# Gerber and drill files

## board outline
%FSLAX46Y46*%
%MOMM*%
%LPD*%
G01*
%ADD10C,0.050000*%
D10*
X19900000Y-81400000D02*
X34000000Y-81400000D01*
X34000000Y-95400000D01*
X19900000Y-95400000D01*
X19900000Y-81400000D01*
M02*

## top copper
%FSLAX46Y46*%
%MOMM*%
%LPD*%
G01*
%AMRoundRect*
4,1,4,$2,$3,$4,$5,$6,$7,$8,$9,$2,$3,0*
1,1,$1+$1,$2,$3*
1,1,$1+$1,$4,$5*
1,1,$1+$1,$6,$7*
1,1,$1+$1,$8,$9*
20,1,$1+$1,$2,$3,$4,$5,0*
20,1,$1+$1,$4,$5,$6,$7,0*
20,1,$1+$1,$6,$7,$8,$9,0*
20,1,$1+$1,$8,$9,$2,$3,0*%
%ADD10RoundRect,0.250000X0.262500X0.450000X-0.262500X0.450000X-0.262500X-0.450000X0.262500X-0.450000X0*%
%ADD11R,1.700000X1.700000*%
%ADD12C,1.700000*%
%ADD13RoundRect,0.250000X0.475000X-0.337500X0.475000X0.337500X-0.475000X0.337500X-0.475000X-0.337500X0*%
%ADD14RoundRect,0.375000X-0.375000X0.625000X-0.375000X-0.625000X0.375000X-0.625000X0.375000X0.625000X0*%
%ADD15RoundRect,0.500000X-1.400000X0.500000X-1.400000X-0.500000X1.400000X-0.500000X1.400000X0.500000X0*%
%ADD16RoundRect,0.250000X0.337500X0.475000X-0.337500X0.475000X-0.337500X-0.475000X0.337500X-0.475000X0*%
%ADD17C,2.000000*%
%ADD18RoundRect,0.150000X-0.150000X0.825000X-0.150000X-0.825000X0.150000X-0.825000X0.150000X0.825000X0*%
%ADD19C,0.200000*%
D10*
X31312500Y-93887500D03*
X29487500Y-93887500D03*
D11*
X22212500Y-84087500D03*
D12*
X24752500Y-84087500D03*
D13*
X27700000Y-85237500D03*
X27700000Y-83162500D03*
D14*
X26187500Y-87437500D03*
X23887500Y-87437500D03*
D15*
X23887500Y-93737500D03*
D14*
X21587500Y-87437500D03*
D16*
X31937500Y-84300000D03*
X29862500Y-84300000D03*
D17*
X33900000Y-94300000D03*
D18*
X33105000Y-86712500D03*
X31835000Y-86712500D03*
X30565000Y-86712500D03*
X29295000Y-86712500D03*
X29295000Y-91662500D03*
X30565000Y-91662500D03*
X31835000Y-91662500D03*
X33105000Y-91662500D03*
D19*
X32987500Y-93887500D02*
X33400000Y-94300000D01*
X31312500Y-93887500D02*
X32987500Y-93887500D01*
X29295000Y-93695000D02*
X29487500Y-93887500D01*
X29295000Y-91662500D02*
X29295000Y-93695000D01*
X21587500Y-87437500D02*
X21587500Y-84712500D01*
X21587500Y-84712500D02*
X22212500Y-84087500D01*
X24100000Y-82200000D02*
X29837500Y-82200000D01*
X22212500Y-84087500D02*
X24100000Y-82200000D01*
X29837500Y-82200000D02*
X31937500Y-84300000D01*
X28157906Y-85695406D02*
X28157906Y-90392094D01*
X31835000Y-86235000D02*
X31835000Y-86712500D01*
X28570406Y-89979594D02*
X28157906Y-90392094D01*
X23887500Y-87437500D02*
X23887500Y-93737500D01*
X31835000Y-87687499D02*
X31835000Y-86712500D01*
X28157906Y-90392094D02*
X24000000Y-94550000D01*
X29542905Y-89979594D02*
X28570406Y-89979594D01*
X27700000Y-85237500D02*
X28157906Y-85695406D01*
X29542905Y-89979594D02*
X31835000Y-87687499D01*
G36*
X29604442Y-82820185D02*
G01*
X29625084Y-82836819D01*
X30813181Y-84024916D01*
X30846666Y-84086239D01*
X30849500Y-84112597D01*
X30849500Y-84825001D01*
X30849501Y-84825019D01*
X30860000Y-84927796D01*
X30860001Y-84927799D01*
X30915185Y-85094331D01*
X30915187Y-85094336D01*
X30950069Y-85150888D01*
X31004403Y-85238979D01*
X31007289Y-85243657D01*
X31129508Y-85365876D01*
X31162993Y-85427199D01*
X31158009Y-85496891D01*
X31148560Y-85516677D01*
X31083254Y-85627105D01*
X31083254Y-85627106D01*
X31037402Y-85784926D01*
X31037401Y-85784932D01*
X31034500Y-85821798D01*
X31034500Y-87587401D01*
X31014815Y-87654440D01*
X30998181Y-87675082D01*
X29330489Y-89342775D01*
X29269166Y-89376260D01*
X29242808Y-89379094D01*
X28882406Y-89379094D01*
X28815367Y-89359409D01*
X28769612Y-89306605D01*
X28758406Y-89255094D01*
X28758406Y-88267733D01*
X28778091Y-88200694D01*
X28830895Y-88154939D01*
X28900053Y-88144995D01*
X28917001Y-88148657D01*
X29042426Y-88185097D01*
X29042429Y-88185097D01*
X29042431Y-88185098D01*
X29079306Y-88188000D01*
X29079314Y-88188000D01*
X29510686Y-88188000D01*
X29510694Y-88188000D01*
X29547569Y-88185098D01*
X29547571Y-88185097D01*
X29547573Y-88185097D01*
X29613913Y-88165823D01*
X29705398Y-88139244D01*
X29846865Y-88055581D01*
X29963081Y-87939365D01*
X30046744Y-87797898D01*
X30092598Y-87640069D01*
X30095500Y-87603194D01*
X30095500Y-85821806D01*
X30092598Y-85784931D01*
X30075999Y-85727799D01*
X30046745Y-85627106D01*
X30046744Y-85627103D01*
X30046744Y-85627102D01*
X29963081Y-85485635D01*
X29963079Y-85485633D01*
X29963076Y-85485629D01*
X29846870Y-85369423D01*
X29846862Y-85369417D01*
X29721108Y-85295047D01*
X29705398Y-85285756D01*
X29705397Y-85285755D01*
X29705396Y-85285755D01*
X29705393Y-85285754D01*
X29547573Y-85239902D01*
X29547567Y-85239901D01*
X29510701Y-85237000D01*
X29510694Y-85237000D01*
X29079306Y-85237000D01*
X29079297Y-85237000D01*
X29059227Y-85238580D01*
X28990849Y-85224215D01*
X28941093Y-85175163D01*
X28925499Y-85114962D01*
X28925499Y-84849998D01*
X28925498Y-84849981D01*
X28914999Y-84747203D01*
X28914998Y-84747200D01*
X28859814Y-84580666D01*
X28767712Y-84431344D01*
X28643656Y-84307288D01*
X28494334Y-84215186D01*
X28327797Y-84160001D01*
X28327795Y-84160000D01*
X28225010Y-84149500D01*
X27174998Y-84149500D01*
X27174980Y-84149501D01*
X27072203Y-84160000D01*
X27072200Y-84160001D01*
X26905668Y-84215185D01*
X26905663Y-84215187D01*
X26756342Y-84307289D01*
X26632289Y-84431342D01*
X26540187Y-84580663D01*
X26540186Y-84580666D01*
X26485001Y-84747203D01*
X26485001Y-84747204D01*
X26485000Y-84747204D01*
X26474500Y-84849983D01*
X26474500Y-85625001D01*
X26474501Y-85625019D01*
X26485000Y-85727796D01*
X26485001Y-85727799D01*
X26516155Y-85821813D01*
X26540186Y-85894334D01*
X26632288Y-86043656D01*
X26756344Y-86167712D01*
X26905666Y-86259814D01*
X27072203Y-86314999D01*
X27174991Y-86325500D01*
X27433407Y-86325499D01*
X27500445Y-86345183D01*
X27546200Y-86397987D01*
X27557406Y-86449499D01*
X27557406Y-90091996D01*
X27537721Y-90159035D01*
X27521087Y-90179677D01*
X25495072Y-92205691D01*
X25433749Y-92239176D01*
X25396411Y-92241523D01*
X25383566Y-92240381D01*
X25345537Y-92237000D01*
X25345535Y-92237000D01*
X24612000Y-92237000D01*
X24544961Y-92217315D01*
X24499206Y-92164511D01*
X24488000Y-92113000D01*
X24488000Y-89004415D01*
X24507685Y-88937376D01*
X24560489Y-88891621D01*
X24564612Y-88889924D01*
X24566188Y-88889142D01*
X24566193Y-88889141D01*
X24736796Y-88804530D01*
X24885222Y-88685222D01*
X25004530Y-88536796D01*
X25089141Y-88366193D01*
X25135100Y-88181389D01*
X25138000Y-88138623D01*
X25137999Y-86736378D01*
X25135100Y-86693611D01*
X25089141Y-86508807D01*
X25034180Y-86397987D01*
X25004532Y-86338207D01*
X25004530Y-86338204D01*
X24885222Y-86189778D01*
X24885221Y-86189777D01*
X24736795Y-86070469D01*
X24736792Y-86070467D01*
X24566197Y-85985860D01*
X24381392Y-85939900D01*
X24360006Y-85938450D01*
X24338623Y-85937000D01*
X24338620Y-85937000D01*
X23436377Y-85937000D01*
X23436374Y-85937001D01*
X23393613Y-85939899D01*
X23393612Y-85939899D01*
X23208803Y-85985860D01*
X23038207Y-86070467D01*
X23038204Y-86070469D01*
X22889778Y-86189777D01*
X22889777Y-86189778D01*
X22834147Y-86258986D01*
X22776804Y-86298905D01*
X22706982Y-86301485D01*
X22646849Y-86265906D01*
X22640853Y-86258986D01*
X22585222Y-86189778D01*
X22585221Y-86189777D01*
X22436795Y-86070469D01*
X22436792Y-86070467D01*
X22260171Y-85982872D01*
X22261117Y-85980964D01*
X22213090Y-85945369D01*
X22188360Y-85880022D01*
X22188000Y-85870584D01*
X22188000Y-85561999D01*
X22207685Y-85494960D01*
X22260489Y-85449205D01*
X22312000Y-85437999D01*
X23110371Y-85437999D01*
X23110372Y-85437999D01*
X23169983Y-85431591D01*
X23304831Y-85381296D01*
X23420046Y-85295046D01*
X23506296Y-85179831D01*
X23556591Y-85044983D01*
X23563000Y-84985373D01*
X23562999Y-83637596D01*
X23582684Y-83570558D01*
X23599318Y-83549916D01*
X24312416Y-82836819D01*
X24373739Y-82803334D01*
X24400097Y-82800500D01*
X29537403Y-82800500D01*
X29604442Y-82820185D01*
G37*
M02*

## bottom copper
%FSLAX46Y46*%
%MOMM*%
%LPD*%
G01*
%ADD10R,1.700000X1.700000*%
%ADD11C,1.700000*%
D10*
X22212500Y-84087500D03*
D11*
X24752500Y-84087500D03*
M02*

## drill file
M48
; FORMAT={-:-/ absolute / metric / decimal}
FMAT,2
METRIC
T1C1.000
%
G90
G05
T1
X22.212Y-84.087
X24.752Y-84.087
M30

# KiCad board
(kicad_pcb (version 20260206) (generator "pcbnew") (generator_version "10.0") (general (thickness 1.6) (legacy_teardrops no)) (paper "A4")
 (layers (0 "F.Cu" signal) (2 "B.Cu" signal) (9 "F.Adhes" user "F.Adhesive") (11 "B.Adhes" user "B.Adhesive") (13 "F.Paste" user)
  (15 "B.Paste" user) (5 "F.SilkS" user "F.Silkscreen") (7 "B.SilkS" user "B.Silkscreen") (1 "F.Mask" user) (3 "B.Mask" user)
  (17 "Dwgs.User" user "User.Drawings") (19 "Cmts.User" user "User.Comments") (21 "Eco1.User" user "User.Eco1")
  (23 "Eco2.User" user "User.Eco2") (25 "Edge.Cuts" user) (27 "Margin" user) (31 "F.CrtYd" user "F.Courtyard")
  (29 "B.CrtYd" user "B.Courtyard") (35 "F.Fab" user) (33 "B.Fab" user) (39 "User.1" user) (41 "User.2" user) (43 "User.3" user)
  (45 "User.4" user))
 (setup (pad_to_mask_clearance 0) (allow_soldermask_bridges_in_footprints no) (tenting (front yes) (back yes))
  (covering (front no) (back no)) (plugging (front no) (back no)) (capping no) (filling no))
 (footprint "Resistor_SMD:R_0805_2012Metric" (layer "F.Cu") (at 30.4 93.8875 180)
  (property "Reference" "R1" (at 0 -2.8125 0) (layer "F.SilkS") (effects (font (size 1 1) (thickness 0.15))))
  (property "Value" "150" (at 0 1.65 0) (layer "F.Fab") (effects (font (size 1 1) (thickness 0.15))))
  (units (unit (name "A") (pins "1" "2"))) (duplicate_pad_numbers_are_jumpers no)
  (pad "1" smd roundrect (at -0.9125 0 180) (size 1.025 1.4) (layers "F.Cu" "F.Mask" "F.Paste") (roundrect_rratio 0.243902) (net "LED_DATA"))
  (pad "2" smd roundrect (at 0.9125 0 180) (size 1.025 1.4) (layers "F.Cu" "F.Mask" "F.Paste") (roundrect_rratio 0.243902)
   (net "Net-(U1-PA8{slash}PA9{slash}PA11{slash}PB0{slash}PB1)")))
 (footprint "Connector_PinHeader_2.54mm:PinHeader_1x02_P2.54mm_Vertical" (layer "F.Cu") (at 22.2125 84.0875 90)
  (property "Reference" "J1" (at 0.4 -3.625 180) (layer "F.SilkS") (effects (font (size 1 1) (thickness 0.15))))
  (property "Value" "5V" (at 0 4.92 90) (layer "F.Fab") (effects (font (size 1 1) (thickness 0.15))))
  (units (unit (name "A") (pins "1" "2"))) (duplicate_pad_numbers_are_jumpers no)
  (pad "1" thru_hole rect (at 0 0 90) (size 1.7 1.7) (drill 1) (layers "*.Cu" "*.Mask") (remove_unused_layers no) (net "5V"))
  (pad "2" thru_hole circle (at 0 2.54 90) (size 1.7 1.7) (drill 1) (layers "*.Cu" "*.Mask") (remove_unused_layers no) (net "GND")))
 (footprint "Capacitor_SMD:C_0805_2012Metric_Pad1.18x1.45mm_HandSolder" (layer "F.Cu") (at 27.7 84.2 90)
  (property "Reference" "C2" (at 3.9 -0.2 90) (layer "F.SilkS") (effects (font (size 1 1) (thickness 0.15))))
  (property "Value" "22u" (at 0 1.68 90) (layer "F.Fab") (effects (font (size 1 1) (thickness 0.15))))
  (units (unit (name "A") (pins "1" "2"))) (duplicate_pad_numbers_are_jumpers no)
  (pad "1" smd roundrect (at -1.0375 0 90) (size 1.175 1.45) (layers "F.Cu" "F.Mask" "F.Paste") (roundrect_rratio 0.212766) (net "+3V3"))
  (pad "2" smd roundrect (at 1.0375 0 90) (size 1.175 1.45) (layers "F.Cu" "F.Mask" "F.Paste") (roundrect_rratio 0.212766) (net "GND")))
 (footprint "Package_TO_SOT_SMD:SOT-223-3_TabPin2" (layer "F.Cu") (at 23.8875 90.5875 -90)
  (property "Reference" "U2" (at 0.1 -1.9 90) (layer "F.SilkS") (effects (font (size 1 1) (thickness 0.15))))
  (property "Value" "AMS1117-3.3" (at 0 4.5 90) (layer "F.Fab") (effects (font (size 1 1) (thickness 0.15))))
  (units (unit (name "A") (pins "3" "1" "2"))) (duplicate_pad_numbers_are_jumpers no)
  (pad "1" smd roundrect (at -3.15 -2.3 270) (size 2 1.5) (layers "F.Cu" "F.Mask" "F.Paste") (roundrect_rratio 0.25) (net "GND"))
  (pad "2" smd roundrect (at -3.15 0 270) (size 2 1.5) (layers "F.Cu" "F.Mask" "F.Paste") (roundrect_rratio 0.25) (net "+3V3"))
  (pad "2" smd roundrect (at 3.15 0 270) (size 2 3.8) (layers "F.Cu" "F.Mask" "F.Paste") (roundrect_rratio 0.25) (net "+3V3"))
  (pad "3" smd roundrect (at -3.15 2.3 270) (size 2 1.5) (layers "F.Cu" "F.Mask" "F.Paste") (roundrect_rratio 0.25) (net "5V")))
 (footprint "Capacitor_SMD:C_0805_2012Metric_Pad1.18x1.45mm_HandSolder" (layer "F.Cu") (at 30.9 84.3 180)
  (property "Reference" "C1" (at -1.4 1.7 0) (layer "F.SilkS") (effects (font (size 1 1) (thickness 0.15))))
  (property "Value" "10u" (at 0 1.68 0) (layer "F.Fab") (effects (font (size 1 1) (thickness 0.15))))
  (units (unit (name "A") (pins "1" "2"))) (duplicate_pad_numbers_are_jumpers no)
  (pad "1" smd roundrect (at -1.0375 0 180) (size 1.175 1.45) (layers "F.Cu" "F.Mask" "F.Paste") (roundrect_rratio 0.212766) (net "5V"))
  (pad "2" smd roundrect (at 1.0375 0 180) (size 1.175 1.45) (layers "F.Cu" "F.Mask" "F.Paste") (roundrect_rratio 0.212766) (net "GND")))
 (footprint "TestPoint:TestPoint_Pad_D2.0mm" (layer "F.Cu") (at 33.9 94.3)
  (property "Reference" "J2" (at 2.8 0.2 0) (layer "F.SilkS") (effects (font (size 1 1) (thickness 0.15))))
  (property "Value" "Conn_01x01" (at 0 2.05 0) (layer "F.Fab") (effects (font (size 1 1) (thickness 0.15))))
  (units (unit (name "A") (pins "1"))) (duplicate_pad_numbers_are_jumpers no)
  (pad "1" smd circle (at 0 0) (size 2 2) (layers "F.Cu" "F.Mask") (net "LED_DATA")))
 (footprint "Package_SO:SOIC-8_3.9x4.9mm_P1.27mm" (layer "F.Cu") (at 31.2 89.1875 -90)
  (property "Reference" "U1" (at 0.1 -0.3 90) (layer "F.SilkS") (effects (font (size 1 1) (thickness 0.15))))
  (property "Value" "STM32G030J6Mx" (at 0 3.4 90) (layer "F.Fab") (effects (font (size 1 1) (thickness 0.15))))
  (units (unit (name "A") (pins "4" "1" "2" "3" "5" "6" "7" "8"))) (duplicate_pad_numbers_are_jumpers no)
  (pad "1" smd roundrect (at -2.475 -1.905 270) (size 1.95 0.6) (layers "F.Cu" "F.Mask" "F.Paste") (roundrect_rratio 0.25)
   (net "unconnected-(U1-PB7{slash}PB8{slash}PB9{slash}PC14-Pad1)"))
  (pad "2" smd roundrect (at -2.475 -0.635 270) (size 1.95 0.6) (layers "F.Cu" "F.Mask" "F.Paste") (roundrect_rratio 0.25) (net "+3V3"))
  (pad "3" smd roundrect (at -2.475 0.635 270) (size 1.95 0.6) (layers "F.Cu" "F.Mask" "F.Paste") (roundrect_rratio 0.25) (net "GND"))
  (pad "4" smd roundrect (at -2.475 1.905 270) (size 1.95 0.6) (layers "F.Cu" "F.Mask" "F.Paste") (roundrect_rratio 0.25)
   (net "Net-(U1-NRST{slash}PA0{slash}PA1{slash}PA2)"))
  (pad "5" smd roundrect (at 2.475 1.905 270) (size 1.95 0.6) (layers "F.Cu" "F.Mask" "F.Paste") (roundrect_rratio 0.25)
   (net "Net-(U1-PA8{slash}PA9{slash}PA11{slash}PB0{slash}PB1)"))
  (pad "6" smd roundrect (at 2.475 0.635 270) (size 1.95 0.6) (layers "F.Cu" "F.Mask" "F.Paste") (roundrect_rratio 0.25)
   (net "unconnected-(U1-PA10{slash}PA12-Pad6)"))
  (pad "7" smd roundrect (at 2.475 -0.635 270) (size 1.95 0.6) (layers "F.Cu" "F.Mask" "F.Paste") (roundrect_rratio 0.25)
   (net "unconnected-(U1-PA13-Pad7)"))
  (pad "8" smd roundrect (at 2.475 -1.905 270) (size 1.95 0.6) (layers "F.Cu" "F.Mask" "F.Paste") (roundrect_rratio 0.25)
   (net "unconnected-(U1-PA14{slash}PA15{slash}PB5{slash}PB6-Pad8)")))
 (gr_rect (start 19.9 81.4) (end 34 95.4) (stroke (width 0.05) (type default)) (fill no) (layer "Edge.Cuts"))
 (segment (start 32.9875 93.8875) (end 33.4 94.3) (width 0.2) (layer "F.Cu") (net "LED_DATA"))
 (segment (start 31.3125 93.8875) (end 32.9875 93.8875) (width 0.2) (layer "F.Cu") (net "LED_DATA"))
 (segment (start 29.295 93.695) (end 29.4875 93.8875) (width 0.2) (layer "F.Cu")
  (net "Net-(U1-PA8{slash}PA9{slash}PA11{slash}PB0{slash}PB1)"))
 (segment (start 29.295 91.6625) (end 29.295 93.695) (width 0.2) (layer "F.Cu")
  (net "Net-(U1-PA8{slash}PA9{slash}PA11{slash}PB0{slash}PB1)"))
 (segment (start 21.5875 87.4375) (end 21.5875 84.7125) (width 0.2) (layer "F.Cu") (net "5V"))
 (segment (start 21.5875 84.7125) (end 22.2125 84.0875) (width 0.2) (layer "F.Cu") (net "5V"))
 (segment (start 24.1 82.2) (end 29.8375 82.2) (width 0.2) (layer "F.Cu") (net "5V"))
 (segment (start 22.2125 84.0875) (end 24.1 82.2) (width 0.2) (layer "F.Cu") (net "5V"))
 (segment (start 29.8375 82.2) (end 31.9375 84.3) (width 0.2) (layer "F.Cu") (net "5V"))
 (segment (start 28.157906 85.695406) (end 28.157906 90.392094) (width 0.2) (layer "F.Cu") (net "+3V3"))
 (segment (start 31.835 86.235) (end 31.835 86.7125) (width 0.2) (layer "F.Cu") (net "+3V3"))
 (segment (start 28.570406 89.979594) (end 28.157906 90.392094) (width 0.2) (layer "F.Cu") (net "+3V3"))
 (segment (start 23.8875 87.4375) (end 23.8875 93.7375) (width 0.2) (layer "F.Cu") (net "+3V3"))
 (segment (start 31.835 87.687499) (end 31.835 86.7125) (width 0.2) (layer "F.Cu") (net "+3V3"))
 (segment (start 28.157906 90.392094) (end 24 94.55) (width 0.2) (layer "F.Cu") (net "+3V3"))
 (segment (start 29.542905 89.979594) (end 28.570406 89.979594) (width 0.2) (layer "F.Cu") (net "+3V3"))
 (segment (start 27.7 85.2375) (end 28.157906 85.695406) (width 0.2) (layer "F.Cu") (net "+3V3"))
 (segment (start 29.542905 89.979594) (end 31.835 87.687499) (width 0.2) (layer "F.Cu") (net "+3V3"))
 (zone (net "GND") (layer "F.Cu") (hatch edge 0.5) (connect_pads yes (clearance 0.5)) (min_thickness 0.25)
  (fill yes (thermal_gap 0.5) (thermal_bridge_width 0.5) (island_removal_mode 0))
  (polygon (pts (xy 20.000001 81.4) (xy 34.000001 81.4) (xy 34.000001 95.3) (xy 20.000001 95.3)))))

